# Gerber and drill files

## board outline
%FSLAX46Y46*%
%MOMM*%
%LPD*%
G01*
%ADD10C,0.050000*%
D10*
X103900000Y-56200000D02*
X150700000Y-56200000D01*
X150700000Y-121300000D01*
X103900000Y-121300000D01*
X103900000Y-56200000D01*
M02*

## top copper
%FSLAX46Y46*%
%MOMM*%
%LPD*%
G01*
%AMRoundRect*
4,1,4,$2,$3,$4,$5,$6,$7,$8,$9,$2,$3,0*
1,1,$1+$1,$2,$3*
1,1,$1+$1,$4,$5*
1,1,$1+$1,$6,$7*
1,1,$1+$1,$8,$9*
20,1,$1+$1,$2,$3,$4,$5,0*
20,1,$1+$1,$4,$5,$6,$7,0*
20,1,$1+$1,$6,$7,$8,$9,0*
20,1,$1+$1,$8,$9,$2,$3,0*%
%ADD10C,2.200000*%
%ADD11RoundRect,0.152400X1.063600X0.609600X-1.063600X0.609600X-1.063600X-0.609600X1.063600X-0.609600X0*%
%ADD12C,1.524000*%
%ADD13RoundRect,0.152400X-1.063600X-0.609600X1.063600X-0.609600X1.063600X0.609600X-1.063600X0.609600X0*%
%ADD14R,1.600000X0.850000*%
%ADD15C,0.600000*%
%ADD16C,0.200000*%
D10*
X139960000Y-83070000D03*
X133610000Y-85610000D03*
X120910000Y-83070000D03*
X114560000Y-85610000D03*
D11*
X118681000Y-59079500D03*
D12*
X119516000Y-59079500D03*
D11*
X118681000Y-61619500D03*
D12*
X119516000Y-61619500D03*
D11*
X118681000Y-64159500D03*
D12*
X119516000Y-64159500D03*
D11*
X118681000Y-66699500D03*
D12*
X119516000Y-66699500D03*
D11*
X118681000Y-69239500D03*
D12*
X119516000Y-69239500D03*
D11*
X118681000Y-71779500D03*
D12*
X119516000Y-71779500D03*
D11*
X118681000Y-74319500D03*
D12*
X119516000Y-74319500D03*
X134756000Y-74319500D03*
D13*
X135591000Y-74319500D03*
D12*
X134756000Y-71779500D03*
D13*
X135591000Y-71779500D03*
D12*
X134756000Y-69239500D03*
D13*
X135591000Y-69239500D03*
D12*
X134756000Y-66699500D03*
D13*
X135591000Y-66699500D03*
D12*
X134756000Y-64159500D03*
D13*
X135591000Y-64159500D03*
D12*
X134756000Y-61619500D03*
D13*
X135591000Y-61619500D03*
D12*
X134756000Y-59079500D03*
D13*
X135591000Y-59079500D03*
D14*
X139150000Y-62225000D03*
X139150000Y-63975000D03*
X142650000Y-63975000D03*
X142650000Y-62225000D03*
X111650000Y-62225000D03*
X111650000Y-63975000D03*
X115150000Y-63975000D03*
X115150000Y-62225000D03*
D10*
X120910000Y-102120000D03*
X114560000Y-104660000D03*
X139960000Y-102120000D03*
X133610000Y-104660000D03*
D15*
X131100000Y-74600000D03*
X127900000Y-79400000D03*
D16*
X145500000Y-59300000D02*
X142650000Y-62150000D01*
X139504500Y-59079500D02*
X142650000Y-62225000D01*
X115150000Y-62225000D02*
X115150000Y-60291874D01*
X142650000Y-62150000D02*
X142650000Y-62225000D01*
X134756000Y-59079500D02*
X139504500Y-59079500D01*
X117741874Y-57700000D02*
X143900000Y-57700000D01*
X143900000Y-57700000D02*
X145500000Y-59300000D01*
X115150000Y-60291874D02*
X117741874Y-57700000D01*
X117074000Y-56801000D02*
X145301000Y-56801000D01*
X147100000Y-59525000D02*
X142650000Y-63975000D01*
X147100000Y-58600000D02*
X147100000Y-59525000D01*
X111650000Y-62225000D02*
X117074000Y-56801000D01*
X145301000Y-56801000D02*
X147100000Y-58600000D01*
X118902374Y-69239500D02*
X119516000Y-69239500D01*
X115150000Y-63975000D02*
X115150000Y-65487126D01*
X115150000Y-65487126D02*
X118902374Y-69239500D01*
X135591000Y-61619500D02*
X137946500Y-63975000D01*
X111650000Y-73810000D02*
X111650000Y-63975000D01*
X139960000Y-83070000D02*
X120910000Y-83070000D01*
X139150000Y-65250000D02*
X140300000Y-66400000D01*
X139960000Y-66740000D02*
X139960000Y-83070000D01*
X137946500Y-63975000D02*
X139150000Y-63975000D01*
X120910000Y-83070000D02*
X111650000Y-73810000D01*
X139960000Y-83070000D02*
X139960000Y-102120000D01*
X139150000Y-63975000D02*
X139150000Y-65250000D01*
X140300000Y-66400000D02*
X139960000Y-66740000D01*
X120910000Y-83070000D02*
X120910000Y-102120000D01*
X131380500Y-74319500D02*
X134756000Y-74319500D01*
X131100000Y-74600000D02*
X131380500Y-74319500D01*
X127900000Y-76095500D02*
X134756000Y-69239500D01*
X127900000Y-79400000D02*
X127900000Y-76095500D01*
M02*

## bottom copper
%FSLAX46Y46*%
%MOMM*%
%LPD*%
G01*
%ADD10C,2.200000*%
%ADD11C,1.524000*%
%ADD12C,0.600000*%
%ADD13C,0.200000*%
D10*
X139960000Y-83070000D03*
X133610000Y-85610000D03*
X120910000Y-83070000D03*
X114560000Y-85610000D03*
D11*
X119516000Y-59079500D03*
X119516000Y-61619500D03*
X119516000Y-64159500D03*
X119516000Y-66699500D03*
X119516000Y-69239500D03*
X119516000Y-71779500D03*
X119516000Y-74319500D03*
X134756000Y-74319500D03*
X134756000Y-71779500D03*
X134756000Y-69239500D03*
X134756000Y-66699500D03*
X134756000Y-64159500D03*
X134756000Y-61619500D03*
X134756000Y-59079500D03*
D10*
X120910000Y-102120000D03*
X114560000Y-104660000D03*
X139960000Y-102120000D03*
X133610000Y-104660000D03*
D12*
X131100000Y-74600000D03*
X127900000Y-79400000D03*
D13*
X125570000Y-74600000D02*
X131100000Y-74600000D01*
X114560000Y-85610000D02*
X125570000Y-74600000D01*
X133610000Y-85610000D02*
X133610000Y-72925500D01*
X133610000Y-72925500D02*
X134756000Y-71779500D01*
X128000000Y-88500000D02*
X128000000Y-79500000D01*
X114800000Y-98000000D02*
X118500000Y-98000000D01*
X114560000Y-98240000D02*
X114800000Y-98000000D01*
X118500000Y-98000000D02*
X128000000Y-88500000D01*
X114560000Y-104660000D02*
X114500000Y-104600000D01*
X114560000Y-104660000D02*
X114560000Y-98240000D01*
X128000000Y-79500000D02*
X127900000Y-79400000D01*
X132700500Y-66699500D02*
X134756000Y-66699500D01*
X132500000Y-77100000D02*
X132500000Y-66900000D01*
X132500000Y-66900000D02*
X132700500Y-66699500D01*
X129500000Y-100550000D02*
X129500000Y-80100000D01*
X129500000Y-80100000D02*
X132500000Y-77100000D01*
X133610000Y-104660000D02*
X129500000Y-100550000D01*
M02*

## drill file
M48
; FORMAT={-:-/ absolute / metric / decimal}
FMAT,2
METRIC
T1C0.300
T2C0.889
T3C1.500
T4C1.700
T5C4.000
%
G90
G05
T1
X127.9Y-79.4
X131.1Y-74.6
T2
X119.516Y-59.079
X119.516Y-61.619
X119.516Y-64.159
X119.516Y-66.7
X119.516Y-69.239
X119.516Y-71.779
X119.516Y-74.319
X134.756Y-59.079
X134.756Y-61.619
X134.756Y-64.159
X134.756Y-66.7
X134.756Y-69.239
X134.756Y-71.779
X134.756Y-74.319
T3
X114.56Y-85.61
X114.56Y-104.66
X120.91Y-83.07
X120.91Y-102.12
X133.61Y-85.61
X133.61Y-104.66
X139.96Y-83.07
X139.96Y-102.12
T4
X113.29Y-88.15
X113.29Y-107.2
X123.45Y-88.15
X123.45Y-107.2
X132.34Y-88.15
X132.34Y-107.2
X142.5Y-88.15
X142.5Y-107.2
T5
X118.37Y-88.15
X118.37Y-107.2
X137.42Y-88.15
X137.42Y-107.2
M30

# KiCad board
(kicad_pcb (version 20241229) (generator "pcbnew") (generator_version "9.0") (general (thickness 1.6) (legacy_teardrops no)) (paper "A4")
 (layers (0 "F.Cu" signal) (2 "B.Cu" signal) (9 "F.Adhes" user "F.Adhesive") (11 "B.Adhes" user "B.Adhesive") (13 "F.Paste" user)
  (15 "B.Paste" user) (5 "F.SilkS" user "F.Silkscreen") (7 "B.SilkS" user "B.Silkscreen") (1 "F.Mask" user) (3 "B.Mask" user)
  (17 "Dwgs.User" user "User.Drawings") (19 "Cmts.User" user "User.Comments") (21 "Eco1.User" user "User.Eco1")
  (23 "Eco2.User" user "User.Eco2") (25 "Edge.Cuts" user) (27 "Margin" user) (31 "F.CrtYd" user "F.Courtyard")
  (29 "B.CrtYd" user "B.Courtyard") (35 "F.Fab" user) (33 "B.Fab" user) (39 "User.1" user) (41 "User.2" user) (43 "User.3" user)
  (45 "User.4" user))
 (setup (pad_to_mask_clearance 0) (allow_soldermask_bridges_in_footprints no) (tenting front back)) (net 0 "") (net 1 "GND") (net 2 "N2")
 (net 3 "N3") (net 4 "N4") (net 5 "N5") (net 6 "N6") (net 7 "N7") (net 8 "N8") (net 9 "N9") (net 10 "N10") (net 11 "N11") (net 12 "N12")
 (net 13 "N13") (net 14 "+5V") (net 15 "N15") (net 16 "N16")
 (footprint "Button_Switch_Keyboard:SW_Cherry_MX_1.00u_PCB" (layer "F.Cu") (at 139.96 83.07)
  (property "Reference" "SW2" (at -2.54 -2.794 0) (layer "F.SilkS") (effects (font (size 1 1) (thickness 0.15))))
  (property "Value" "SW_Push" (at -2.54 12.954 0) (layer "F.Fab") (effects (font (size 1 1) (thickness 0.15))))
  (pad "" np_thru_hole circle (at -7.62 5.08) (size 1.7 1.7) (drill 1.7) (layers "*.Cu" "*.Mask"))
  (pad "" np_thru_hole circle (at -2.54 5.08) (size 4 4) (drill 4) (layers "*.Cu" "*.Mask"))
  (pad "" np_thru_hole circle (at 2.54 5.08) (size 1.7 1.7) (drill 1.7) (layers "*.Cu" "*.Mask"))
  (pad "1" thru_hole circle (at 0 0) (size 2.2 2.2) (drill 1.5) (layers "*.Cu" "*.Mask") (remove_unused_layers no) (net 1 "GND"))
  (pad "2" thru_hole circle (at -6.35 2.54) (size 2.2 2.2) (drill 1.5) (layers "*.Cu" "*.Mask") (remove_unused_layers no) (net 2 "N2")))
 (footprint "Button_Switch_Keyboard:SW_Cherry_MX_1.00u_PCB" (layer "F.Cu") (at 120.91 83.07)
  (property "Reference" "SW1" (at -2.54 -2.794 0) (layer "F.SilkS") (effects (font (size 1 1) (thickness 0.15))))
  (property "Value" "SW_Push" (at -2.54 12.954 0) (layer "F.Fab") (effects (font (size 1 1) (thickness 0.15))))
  (pad "" np_thru_hole circle (at -7.62 5.08) (size 1.7 1.7) (drill 1.7) (layers "*.Cu" "*.Mask"))
  (pad "" np_thru_hole circle (at -2.54 5.08) (size 4 4) (drill 4) (layers "*.Cu" "*.Mask"))
  (pad "" np_thru_hole circle (at 2.54 5.08) (size 1.7 1.7) (drill 1.7) (layers "*.Cu" "*.Mask"))
  (pad "1" thru_hole circle (at 0 0) (size 2.2 2.2) (drill 1.5) (layers "*.Cu" "*.Mask") (remove_unused_layers no) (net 1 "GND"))
  (pad "2" thru_hole circle (at -6.35 2.54) (size 2.2 2.2) (drill 1.5) (layers "*.Cu" "*.Mask") (remove_unused_layers no) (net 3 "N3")))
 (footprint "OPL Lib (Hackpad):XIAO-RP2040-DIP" (layer "F.Cu") (at 127.136 66.6995)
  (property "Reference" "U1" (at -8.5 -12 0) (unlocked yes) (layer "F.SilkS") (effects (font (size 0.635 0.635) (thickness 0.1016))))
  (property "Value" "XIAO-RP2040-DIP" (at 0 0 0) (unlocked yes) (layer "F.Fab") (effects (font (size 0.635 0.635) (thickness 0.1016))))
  (pad "1" smd roundrect (at -8.455 -7.62 180) (size 2.432 1.524) (layers "F.Cu" "F.Mask") (roundrect_rratio 0.1) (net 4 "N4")
   (thermal_bridge_angle 45))
  (pad "1" thru_hole circle (at -7.62 -7.62 180) (size 1.524 1.524) (drill 0.889) (layers "*.Cu" "*.Mask") (remove_unused_layers no)
   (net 4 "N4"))
  (pad "2" smd roundrect (at -8.455 -5.08 180) (size 2.432 1.524) (layers "F.Cu" "F.Mask") (roundrect_rratio 0.1) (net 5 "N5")
   (thermal_bridge_angle 45))
  (pad "2" thru_hole circle (at -7.62 -5.08 180) (size 1.524 1.524) (drill 0.889) (layers "*.Cu" "*.Mask") (remove_unused_layers no)
   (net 5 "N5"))
  (pad "3" smd roundrect (at -8.455 -2.54 180) (size 2.432 1.524) (layers "F.Cu" "F.Mask") (roundrect_rratio 0.1) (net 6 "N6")
   (thermal_bridge_angle 45))
  (pad "3" thru_hole circle (at -7.62 -2.54 180) (size 1.524 1.524) (drill 0.889) (layers "*.Cu" "*.Mask") (remove_unused_layers no)
   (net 6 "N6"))
  (pad "4" smd roundrect (at -8.455 0 180) (size 2.432 1.524) (layers "F.Cu" "F.Mask") (roundrect_rratio 0.1) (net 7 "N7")
   (thermal_bridge_angle 45))
  (pad "4" thru_hole circle (at -7.62 0 180) (size 1.524 1.524) (drill 0.889) (layers "*.Cu" "*.Mask") (remove_unused_layers no)
   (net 7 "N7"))
  (pad "5" smd roundrect (at -8.455 2.54 180) (size 2.432 1.524) (layers "F.Cu" "F.Mask") (roundrect_rratio 0.1) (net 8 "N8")
   (thermal_bridge_angle 45))
  (pad "5" thru_hole circle (at -7.62 2.54 180) (size 1.524 1.524) (drill 0.889) (layers "*.Cu" "*.Mask") (remove_unused_layers no)
   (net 8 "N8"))
  (pad "6" smd roundrect (at -8.455 5.08 180) (size 2.432 1.524) (layers "F.Cu" "F.Mask") (roundrect_rratio 0.1) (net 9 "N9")
   (thermal_bridge_angle 45))
  (pad "6" thru_hole circle (at -7.62 5.08 180) (size 1.524 1.524) (drill 0.889) (layers "*.Cu" "*.Mask") (remove_unused_layers no)
   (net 9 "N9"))
  (pad "7" smd roundrect (at -8.455 7.62 180) (size 2.432 1.524) (layers "F.Cu" "F.Mask") (roundrect_rratio 0.1) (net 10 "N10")
   (thermal_bridge_angle 45))
  (pad "7" thru_hole circle (at -7.62 7.62 180) (size 1.524 1.524) (drill 0.889) (layers "*.Cu" "*.Mask") (remove_unused_layers no)
   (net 10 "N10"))
  (pad "8" thru_hole circle (at 7.62 7.62) (size 1.524 1.524) (drill 0.889) (layers "*.Cu" "*.Mask") (remove_unused_layers no) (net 3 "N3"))
  (pad "8" smd roundrect (at 8.455 7.62) (size 2.432 1.524) (layers "F.Cu" "F.Mask") (roundrect_rratio 0.1) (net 3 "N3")
   (thermal_bridge_angle 45))
  (pad "9" thru_hole circle (at 7.62 5.08) (size 1.524 1.524) (drill 0.889) (layers "*.Cu" "*.Mask") (remove_unused_layers no) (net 2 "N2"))
  (pad "9" smd roundrect (at 8.455 5.08) (size 2.432 1.524) (layers "F.Cu" "F.Mask") (roundrect_rratio 0.1) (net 2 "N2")
   (thermal_bridge_angle 45))
  (pad "10" thru_hole circle (at 7.62 2.54) (size 1.524 1.524) (drill 0.889) (layers "*.Cu" "*.Mask") (remove_unused_layers no)
   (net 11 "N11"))
  (pad "10" smd roundrect (at 8.455 2.54) (size 2.432 1.524) (layers "F.Cu" "F.Mask") (roundrect_rratio 0.1) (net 11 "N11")
   (thermal_bridge_angle 45))
  (pad "11" thru_hole circle (at 7.62 0) (size 1.524 1.524) (drill 0.889) (layers "*.Cu" "*.Mask") (remove_unused_layers no) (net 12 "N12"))
  (pad "11" smd roundrect (at 8.455 0) (size 2.432 1.524) (layers "F.Cu" "F.Mask") (roundrect_rratio 0.1) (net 12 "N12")
   (thermal_bridge_angle 45))
  (pad "12" thru_hole circle (at 7.62 -2.54) (size 1.524 1.524) (drill 0.889) (layers "*.Cu" "*.Mask") (remove_unused_layers no)
   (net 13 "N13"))
  (pad "12" smd roundrect (at 8.455 -2.54) (size 2.432 1.524) (layers "F.Cu" "F.Mask") (roundrect_rratio 0.1) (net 13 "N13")
   (thermal_bridge_angle 45))
  (pad "13" thru_hole circle (at 7.62 -5.08) (size 1.524 1.524) (drill 0.889) (layers "*.Cu" "*.Mask") (remove_unused_layers no)
   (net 1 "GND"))
  (pad "13" smd roundrect (at 8.455 -5.08) (size 2.432 1.524) (layers "F.Cu" "F.Mask") (roundrect_rratio 0.1) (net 1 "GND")
   (thermal_bridge_angle 45))
  (pad "14" thru_hole circle (at 7.62 -7.62) (size 1.524 1.524) (drill 0.889) (layers "*.Cu" "*.Mask") (remove_unused_layers no)
   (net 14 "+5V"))
  (pad "14" smd roundrect (at 8.455 -7.62) (size 2.432 1.524) (layers "F.Cu" "F.Mask") (roundrect_rratio 0.1) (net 14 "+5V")
   (thermal_bridge_angle 45)))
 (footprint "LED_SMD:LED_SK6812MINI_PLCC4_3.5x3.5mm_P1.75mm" (layer "F.Cu") (at 140.9 63.1)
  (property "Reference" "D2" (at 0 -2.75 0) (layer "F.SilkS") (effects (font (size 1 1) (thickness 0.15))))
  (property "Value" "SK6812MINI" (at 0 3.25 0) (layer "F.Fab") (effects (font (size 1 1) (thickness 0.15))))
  (pad "1" smd rect (at -1.75 -0.875) (size 1.6 0.85) (layers "F.Cu" "F.Mask" "F.Paste") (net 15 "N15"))
  (pad "2" smd rect (at -1.75 0.875) (size 1.6 0.85) (layers "F.Cu" "F.Mask" "F.Paste") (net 1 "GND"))
  (pad "3" smd rect (at 1.75 0.875) (size 1.6 0.85) (layers "F.Cu" "F.Mask" "F.Paste") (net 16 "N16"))
  (pad "4" smd rect (at 1.75 -0.875) (size 1.6 0.85) (layers "F.Cu" "F.Mask" "F.Paste") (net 14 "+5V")))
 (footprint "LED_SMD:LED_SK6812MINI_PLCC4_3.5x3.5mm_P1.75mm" (layer "F.Cu") (at 113.4 63.1)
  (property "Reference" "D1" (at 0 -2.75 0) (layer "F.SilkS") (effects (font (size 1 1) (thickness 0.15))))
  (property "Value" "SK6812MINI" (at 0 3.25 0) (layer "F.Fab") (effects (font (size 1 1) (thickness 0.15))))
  (pad "1" smd rect (at -1.75 -0.875) (size 1.6 0.85) (layers "F.Cu" "F.Mask" "F.Paste") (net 16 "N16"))
  (pad "2" smd rect (at -1.75 0.875) (size 1.6 0.85) (layers "F.Cu" "F.Mask" "F.Paste") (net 1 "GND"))
  (pad "3" smd rect (at 1.75 0.875) (size 1.6 0.85) (layers "F.Cu" "F.Mask" "F.Paste") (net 8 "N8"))
  (pad "4" smd rect (at 1.75 -0.875) (size 1.6 0.85) (layers "F.Cu" "F.Mask" "F.Paste") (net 14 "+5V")))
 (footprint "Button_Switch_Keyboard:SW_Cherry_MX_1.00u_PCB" (layer "F.Cu") (at 120.91 102.12)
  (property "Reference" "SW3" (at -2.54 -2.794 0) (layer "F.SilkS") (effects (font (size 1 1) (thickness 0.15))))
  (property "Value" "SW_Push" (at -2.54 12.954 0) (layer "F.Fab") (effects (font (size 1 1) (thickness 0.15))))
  (pad "" np_thru_hole circle (at -7.62 5.08) (size 1.7 1.7) (drill 1.7) (layers "*.Cu" "*.Mask"))
  (pad "" np_thru_hole circle (at -2.54 5.08) (size 4 4) (drill 4) (layers "*.Cu" "*.Mask"))
  (pad "" np_thru_hole circle (at 2.54 5.08) (size 1.7 1.7) (drill 1.7) (layers "*.Cu" "*.Mask"))
  (pad "1" thru_hole circle (at 0 0) (size 2.2 2.2) (drill 1.5) (layers "*.Cu" "*.Mask") (remove_unused_layers no) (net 1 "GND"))
  (pad "2" thru_hole circle (at -6.35 2.54) (size 2.2 2.2) (drill 1.5) (layers "*.Cu" "*.Mask") (remove_unused_layers no) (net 11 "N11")))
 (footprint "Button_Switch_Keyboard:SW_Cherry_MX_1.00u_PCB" (layer "F.Cu") (at 139.96 102.12)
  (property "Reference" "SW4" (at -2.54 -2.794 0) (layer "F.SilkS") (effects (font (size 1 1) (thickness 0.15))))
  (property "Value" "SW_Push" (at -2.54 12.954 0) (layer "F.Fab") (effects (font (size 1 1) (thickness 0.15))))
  (pad "" np_thru_hole circle (at -7.62 5.08) (size 1.7 1.7) (drill 1.7) (layers "*.Cu" "*.Mask"))
  (pad "" np_thru_hole circle (at -2.54 5.08) (size 4 4) (drill 4) (layers "*.Cu" "*.Mask"))
  (pad "" np_thru_hole circle (at 2.54 5.08) (size 1.7 1.7) (drill 1.7) (layers "*.Cu" "*.Mask"))
  (pad "1" thru_hole circle (at 0 0) (size 2.2 2.2) (drill 1.5) (layers "*.Cu" "*.Mask") (remove_unused_layers no) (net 1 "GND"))
  (pad "2" thru_hole circle (at -6.35 2.54) (size 2.2 2.2) (drill 1.5) (layers "*.Cu" "*.Mask") (remove_unused_layers no) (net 12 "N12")))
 (gr_rect (start 103.9 56.2) (end 150.7 121.3) (stroke (width 0.05) (type default)) (fill no) (layer "Edge.Cuts"))
 (segment (start 145.5 59.3) (end 142.65 62.15) (width 0.2) (layer "F.Cu") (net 14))
 (segment (start 139.5045 59.0795) (end 142.65 62.225) (width 0.2) (layer "F.Cu") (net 14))
 (segment (start 115.15 62.225) (end 115.15 60.291874) (width 0.2) (layer "F.Cu") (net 14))
 (segment (start 142.65 62.15) (end 142.65 62.225) (width 0.2) (layer "F.Cu") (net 14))
 (segment (start 134.756 59.0795) (end 139.5045 59.0795) (width 0.2) (layer "F.Cu") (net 14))
 (segment (start 117.741874 57.7) (end 143.9 57.7) (width 0.2) (layer "F.Cu") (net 14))
 (segment (start 143.9 57.7) (end 145.5 59.3) (width 0.2) (layer "F.Cu") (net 14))
 (segment (start 115.15 60.291874) (end 117.741874 57.7) (width 0.2) (layer "F.Cu") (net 14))
 (segment (start 117.074 56.801) (end 145.301 56.801) (width 0.2) (layer "F.Cu") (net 16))
 (segment (start 147.1 59.525) (end 142.65 63.975) (width 0.2) (layer "F.Cu") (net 16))
 (segment (start 147.1 58.6) (end 147.1 59.525) (width 0.2) (layer "F.Cu") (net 16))
 (segment (start 111.65 62.225) (end 117.074 56.801) (width 0.2) (layer "F.Cu") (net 16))
 (segment (start 145.301 56.801) (end 147.1 58.6) (width 0.2) (layer "F.Cu") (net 16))
 (segment (start 118.902374 69.2395) (end 119.516 69.2395) (width 0.2) (layer "F.Cu") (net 8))
 (segment (start 115.15 63.975) (end 115.15 65.487126) (width 0.2) (layer "F.Cu") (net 8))
 (segment (start 115.15 65.487126) (end 118.902374 69.2395) (width 0.2) (layer "F.Cu") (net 8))
 (segment (start 135.591 61.6195) (end 137.9465 63.975) (width 0.2) (layer "F.Cu") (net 1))
 (segment (start 111.65 73.81) (end 111.65 63.975) (width 0.2) (layer "F.Cu") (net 1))
 (segment (start 139.96 83.07) (end 120.91 83.07) (width 0.2) (layer "F.Cu") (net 1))
 (segment (start 139.15 65.25) (end 140.3 66.4) (width 0.2) (layer "F.Cu") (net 1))
 (segment (start 139.96 66.74) (end 139.96 83.07) (width 0.2) (layer "F.Cu") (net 1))
 (segment (start 137.9465 63.975) (end 139.15 63.975) (width 0.2) (layer "F.Cu") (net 1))
 (segment (start 120.91 83.07) (end 111.65 73.81) (width 0.2) (layer "F.Cu") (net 1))
 (segment (start 139.96 83.07) (end 139.96 102.12) (width 0.2) (layer "F.Cu") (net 1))
 (segment (start 139.15 63.975) (end 139.15 65.25) (width 0.2) (layer "F.Cu") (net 1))
 (segment (start 140.3 66.4) (end 139.96 66.74) (width 0.2) (layer "F.Cu") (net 1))
 (segment (start 120.91 83.07) (end 120.91 102.12) (width 0.2) (layer "F.Cu") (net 1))
 (segment (start 131.3805 74.3195) (end 134.756 74.3195) (width 0.2) (layer "F.Cu") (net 3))
 (segment (start 131.1 74.6) (end 131.3805 74.3195) (width 0.2) (layer "F.Cu") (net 3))
 (via (at 131.1 74.6) (size 0.6) (drill 0.3) (layers "F.Cu" "B.Cu") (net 3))
 (segment (start 125.57 74.6) (end 131.1 74.6) (width 0.2) (layer "B.Cu") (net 3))
 (segment (start 114.56 85.61) (end 125.57 74.6) (width 0.2) (layer "B.Cu") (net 3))
 (segment (start 133.61 85.61) (end 133.61 72.9255) (width 0.2) (layer "B.Cu") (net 2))
 (segment (start 133.61 72.9255) (end 134.756 71.7795) (width 0.2) (layer "B.Cu") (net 2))
 (segment (start 127.9 76.0955) (end 134.756 69.2395) (width 0.2) (layer "F.Cu") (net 11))
 (segment (start 127.9 79.4) (end 127.9 76.0955) (width 0.2) (layer "F.Cu") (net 11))
 (via (at 127.9 79.4) (size 0.6) (drill 0.3) (layers "F.Cu" "B.Cu") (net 11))
 (segment (start 128 88.5) (end 128 79.5) (width 0.2) (layer "B.Cu") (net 11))
 (segment (start 114.8 98) (end 118.5 98) (width 0.2) (layer "B.Cu") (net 11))
 (segment (start 114.56 98.24) (end 114.8 98) (width 0.2) (layer "B.Cu") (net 11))
 (segment (start 118.5 98) (end 128 88.5) (width 0.2) (layer "B.Cu") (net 11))
 (segment (start 114.56 104.66) (end 114.5 104.6) (width 0.2) (layer "B.Cu") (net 11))
 (segment (start 114.56 104.66) (end 114.56 98.24) (width 0.2) (layer "B.Cu") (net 11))
 (segment (start 128 79.5) (end 127.9 79.4) (width 0.2) (layer "B.Cu") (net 11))
 (segment (start 132.7005 66.6995) (end 134.756 66.6995) (width 0.2) (layer "B.Cu") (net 12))
 (segment (start 132.5 77.1) (end 132.5 66.9) (width 0.2) (layer "B.Cu") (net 12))
 (segment (start 132.5 66.9) (end 132.7005 66.6995) (width 0.2) (layer "B.Cu") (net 12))
 (segment (start 129.5 100.55) (end 129.5 80.1) (width 0.2) (layer "B.Cu") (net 12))
 (segment (start 129.5 80.1) (end 132.5 77.1) (width 0.2) (layer "B.Cu") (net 12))
 (segment (start 133.61 104.66) (end 129.5 100.55) (width 0.2) (layer "B.Cu") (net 12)))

